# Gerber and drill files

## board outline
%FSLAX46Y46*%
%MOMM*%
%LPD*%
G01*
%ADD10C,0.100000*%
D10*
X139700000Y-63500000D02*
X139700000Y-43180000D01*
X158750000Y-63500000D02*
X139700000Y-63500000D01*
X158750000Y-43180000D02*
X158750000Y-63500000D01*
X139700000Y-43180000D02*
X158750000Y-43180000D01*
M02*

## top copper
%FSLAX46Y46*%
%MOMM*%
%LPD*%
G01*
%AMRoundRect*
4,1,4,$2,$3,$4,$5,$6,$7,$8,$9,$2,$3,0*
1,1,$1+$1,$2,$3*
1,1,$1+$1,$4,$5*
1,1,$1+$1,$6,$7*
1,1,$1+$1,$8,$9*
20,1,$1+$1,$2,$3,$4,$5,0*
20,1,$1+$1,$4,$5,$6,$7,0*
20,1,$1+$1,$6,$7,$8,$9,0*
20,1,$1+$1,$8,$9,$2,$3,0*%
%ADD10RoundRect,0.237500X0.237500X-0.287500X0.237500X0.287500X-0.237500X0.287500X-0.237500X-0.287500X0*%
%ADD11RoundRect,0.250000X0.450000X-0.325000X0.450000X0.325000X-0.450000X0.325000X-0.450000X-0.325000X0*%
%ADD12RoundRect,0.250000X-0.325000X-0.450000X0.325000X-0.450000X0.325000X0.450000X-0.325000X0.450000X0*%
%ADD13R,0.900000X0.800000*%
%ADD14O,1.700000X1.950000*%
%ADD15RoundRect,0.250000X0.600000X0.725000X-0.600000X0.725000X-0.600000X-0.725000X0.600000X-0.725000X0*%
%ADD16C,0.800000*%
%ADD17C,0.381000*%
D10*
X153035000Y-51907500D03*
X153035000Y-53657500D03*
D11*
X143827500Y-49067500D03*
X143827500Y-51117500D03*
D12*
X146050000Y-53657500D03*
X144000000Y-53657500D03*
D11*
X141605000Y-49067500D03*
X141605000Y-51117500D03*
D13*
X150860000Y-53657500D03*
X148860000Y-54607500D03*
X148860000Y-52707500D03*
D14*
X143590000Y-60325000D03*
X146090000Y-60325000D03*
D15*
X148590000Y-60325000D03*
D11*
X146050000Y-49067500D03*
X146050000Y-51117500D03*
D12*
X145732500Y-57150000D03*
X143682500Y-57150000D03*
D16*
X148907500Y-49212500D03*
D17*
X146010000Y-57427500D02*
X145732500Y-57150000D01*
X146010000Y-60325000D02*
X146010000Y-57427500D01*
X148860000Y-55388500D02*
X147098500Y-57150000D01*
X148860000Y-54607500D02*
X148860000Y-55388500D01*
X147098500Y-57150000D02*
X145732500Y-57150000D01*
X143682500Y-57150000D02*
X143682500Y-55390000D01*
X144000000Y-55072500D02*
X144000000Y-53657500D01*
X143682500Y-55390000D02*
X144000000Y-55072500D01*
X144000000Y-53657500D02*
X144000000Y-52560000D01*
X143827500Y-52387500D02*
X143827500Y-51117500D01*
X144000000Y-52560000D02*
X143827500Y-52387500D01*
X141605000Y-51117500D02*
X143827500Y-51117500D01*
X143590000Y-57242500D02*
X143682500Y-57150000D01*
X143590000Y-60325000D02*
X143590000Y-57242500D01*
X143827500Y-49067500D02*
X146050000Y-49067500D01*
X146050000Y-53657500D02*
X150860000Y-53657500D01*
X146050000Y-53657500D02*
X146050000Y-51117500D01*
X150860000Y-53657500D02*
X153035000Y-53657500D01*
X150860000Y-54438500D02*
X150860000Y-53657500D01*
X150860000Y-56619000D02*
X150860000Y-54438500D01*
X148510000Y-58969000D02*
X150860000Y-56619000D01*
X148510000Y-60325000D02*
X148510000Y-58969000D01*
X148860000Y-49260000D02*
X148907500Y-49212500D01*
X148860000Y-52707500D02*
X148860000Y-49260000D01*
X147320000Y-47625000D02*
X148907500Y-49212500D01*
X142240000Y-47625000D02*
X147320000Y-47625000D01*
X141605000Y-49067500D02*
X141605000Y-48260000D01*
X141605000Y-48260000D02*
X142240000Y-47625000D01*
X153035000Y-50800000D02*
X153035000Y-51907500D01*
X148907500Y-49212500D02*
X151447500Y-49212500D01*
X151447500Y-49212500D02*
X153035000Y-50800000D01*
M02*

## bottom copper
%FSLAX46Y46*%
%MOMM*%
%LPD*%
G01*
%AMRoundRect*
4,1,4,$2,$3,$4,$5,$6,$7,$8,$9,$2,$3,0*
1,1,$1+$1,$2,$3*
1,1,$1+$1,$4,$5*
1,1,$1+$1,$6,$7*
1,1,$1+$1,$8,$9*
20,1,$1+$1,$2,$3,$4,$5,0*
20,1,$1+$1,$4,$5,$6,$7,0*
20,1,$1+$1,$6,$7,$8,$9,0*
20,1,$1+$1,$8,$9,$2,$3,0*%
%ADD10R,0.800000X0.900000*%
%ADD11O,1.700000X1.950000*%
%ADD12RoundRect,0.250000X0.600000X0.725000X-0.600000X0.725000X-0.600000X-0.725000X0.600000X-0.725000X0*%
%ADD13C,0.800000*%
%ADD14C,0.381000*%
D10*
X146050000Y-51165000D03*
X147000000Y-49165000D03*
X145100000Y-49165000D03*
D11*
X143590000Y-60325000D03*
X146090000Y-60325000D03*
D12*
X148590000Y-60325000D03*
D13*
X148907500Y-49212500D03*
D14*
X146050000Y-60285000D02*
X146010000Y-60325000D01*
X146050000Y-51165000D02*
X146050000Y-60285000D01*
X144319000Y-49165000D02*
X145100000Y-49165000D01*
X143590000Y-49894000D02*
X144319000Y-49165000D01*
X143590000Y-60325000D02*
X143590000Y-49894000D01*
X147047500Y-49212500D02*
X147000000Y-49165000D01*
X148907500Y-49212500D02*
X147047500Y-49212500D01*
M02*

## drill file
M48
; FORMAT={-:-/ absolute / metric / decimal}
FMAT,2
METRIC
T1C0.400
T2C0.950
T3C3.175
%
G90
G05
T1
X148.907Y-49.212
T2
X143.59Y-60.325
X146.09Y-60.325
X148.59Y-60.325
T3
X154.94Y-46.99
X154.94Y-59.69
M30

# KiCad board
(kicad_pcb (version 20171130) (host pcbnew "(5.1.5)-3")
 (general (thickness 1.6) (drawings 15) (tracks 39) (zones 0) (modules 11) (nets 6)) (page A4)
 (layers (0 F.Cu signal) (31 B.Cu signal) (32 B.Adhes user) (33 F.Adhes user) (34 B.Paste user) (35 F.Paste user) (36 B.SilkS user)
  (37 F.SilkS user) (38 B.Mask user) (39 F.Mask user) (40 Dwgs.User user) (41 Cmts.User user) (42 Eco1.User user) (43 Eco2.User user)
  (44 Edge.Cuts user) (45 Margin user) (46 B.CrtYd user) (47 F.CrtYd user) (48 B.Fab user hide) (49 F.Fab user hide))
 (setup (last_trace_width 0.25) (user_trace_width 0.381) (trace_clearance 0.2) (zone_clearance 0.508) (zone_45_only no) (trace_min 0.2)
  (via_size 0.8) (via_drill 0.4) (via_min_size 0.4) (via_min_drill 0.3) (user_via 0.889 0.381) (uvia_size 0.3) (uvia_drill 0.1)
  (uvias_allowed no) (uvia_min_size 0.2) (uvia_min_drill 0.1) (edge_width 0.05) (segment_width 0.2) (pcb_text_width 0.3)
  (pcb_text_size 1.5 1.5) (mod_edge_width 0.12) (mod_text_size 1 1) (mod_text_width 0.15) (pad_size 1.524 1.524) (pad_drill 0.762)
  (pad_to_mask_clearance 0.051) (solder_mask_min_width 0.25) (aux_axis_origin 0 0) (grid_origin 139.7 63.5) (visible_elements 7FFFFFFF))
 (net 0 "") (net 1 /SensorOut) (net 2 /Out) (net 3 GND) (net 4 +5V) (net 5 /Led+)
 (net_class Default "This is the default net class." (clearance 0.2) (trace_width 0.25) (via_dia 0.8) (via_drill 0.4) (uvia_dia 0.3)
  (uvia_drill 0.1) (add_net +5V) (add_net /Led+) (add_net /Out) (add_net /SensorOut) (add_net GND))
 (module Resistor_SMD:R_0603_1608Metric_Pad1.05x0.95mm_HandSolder (layer F.Cu) (at 153.035 52.7825 90)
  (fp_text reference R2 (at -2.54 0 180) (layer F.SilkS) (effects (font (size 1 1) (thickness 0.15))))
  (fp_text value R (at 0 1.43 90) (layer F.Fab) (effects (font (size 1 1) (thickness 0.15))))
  (pad 2 smd roundrect (at 0.875 0 90) (size 1.05 0.95) (layers F.Cu F.Paste F.Mask) (roundrect_rratio 0.25) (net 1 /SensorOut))
  (pad 1 smd roundrect (at -0.875 0 90) (size 1.05 0.95) (layers F.Cu F.Paste F.Mask) (roundrect_rratio 0.25) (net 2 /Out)))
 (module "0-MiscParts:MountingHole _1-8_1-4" (layer F.Cu) (at 154.94 59.69)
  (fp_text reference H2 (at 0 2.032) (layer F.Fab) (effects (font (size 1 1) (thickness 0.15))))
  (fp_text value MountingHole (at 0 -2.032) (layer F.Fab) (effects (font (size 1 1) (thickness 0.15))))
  (pad "" np_thru_hole circle (at 0 0) (size 3.175 3.175) (drill 3.175) (layers *.Cu *.Mask)))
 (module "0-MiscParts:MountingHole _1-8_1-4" (layer F.Cu) (at 154.94 46.99)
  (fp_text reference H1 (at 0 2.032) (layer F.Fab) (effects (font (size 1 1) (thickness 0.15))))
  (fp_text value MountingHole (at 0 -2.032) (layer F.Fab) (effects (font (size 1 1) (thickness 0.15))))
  (pad "" np_thru_hole circle (at 0 0) (size 3.175 3.175) (drill 3.175) (layers *.Cu *.Mask)))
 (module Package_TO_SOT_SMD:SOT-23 (layer B.Cu) (at 146.05 50.165 270)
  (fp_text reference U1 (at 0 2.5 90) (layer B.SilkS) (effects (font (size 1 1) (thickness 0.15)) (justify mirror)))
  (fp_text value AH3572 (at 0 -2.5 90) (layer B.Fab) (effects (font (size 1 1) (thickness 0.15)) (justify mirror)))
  (pad 3 smd rect (at 1 0 270) (size 0.9 0.8) (layers B.Cu B.Paste B.Mask) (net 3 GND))
  (pad 2 smd rect (at -1 -0.95 270) (size 0.9 0.8) (layers B.Cu B.Paste B.Mask) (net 1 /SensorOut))
  (pad 1 smd rect (at -1 0.95 270) (size 0.9 0.8) (layers B.Cu B.Paste B.Mask) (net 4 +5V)))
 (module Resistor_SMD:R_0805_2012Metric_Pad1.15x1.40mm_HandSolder (layer F.Cu) (at 143.8275 50.0925 90)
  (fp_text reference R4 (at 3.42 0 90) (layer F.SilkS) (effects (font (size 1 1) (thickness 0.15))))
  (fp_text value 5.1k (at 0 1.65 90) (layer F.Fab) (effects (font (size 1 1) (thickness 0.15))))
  (pad 2 smd roundrect (at 1.025 0 90) (size 1.15 1.4) (layers F.Cu F.Paste F.Mask) (roundrect_rratio 0.217391) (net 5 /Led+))
  (pad 1 smd roundrect (at -1.025 0 90) (size 1.15 1.4) (layers F.Cu F.Paste F.Mask) (roundrect_rratio 0.217391) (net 4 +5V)))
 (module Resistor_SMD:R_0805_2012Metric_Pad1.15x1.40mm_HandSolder (layer F.Cu) (at 145.025 53.6575)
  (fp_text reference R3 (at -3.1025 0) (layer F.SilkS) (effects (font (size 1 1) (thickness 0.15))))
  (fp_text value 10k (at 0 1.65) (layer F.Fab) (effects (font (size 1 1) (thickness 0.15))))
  (pad 2 smd roundrect (at 1.025 0) (size 1.15 1.4) (layers F.Cu F.Paste F.Mask) (roundrect_rratio 0.217391) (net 2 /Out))
  (pad 1 smd roundrect (at -1.025 0) (size 1.15 1.4) (layers F.Cu F.Paste F.Mask) (roundrect_rratio 0.217391) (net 4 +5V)))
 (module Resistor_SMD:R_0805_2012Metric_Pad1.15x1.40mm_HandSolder (layer F.Cu) (at 141.605 50.0925 90)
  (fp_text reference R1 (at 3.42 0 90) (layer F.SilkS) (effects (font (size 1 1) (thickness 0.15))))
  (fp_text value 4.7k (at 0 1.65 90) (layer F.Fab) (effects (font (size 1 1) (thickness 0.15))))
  (pad 2 smd roundrect (at 1.025 0 90) (size 1.15 1.4) (layers F.Cu F.Paste F.Mask) (roundrect_rratio 0.217391) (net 1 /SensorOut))
  (pad 1 smd roundrect (at -1.025 0 90) (size 1.15 1.4) (layers F.Cu F.Paste F.Mask) (roundrect_rratio 0.217391) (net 4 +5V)))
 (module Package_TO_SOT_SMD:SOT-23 (layer F.Cu) (at 149.86 53.6575)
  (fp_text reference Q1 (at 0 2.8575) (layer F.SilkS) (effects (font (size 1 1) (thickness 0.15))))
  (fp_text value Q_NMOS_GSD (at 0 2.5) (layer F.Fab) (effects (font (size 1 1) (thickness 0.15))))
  (pad 3 smd rect (at 1 0) (size 0.9 0.8) (layers F.Cu F.Paste F.Mask) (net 2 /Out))
  (pad 2 smd rect (at -1 0.95) (size 0.9 0.8) (layers F.Cu F.Paste F.Mask) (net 3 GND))
  (pad 1 smd rect (at -1 -0.95) (size 0.9 0.8) (layers F.Cu F.Paste F.Mask) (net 1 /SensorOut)))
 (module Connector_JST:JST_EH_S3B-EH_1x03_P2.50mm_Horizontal (layer F.Cu) (at 148.59 60.325 180)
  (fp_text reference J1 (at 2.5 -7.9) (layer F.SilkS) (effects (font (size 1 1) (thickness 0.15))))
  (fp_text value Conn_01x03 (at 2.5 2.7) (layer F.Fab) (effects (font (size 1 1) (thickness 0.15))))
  (pad 3 thru_hole oval (at 5 0 180) (size 1.7 1.95) (drill 0.95) (layers *.Cu *.Mask) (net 4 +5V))
  (pad 2 thru_hole oval (at 2.5 0 180) (size 1.7 1.95) (drill 0.95) (layers *.Cu *.Mask) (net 3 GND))
  (pad 1 thru_hole roundrect (at 0 0 180) (size 1.7 1.95) (drill 0.95) (layers *.Cu *.Mask) (roundrect_rratio 0.147059) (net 2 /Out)))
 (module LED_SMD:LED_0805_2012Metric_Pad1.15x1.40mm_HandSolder (layer F.Cu) (at 146.05 50.0925 90)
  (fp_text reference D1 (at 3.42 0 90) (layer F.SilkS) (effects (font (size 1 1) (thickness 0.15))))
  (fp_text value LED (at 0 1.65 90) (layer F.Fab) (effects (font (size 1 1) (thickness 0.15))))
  (pad 2 smd roundrect (at 1.025 0 90) (size 1.15 1.4) (layers F.Cu F.Paste F.Mask) (roundrect_rratio 0.217391) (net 5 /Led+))
  (pad 1 smd roundrect (at -1.025 0 90) (size 1.15 1.4) (layers F.Cu F.Paste F.Mask) (roundrect_rratio 0.217391) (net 2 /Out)))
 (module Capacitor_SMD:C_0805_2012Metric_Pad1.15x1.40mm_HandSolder (layer F.Cu) (at 144.7075 57.15)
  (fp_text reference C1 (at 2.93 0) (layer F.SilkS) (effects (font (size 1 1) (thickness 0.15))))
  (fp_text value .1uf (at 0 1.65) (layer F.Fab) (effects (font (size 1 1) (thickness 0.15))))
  (pad 2 smd roundrect (at 1.025 0) (size 1.15 1.4) (layers F.Cu F.Paste F.Mask) (roundrect_rratio 0.217391) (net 3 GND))
  (pad 1 smd roundrect (at -1.025 0) (size 1.15 1.4) (layers F.Cu F.Paste F.Mask) (roundrect_rratio 0.217391) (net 4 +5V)))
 (gr_line (start 139.7 63.5) (end 139.7 43.18) (layer Edge.Cuts) (width 0.1))
 (gr_line (start 158.75 63.5) (end 139.7 63.5) (layer Edge.Cuts) (width 0.1))
 (gr_line (start 158.75 43.18) (end 158.75 63.5) (layer Edge.Cuts) (width 0.1))
 (gr_line (start 139.7 43.18) (end 158.75 43.18) (layer Edge.Cuts) (width 0.1))
 (segment (start 146.01 57.4275) (end 145.7325 57.15) (width 0.381) (layer F.Cu) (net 3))
 (segment (start 146.01 60.325) (end 146.01 57.4275) (width 0.381) (layer F.Cu) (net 3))
 (segment (start 148.86 55.3885) (end 147.0985 57.15) (width 0.381) (layer F.Cu) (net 3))
 (segment (start 148.86 54.6075) (end 148.86 55.3885) (width 0.381) (layer F.Cu) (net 3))
 (segment (start 147.0985 57.15) (end 145.7325 57.15) (width 0.381) (layer F.Cu) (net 3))
 (segment (start 146.05 60.285) (end 146.01 60.325) (width 0.381) (layer B.Cu) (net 3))
 (segment (start 146.05 51.165) (end 146.05 60.285) (width 0.381) (layer B.Cu) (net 3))
 (segment (start 143.6825 57.15) (end 143.6825 55.39) (width 0.381) (layer F.Cu) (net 4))
 (segment (start 144 55.0725) (end 144 53.6575) (width 0.381) (layer F.Cu) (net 4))
 (segment (start 143.6825 55.39) (end 144 55.0725) (width 0.381) (layer F.Cu) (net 4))
 (segment (start 144 53.6575) (end 144 52.56) (width 0.381) (layer F.Cu) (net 4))
 (segment (start 143.8275 52.3875) (end 143.8275 51.1175) (width 0.381) (layer F.Cu) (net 4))
 (segment (start 144 52.56) (end 143.8275 52.3875) (width 0.381) (layer F.Cu) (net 4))
 (segment (start 141.605 51.1175) (end 143.8275 51.1175) (width 0.381) (layer F.Cu) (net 4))
 (segment (start 144.319 49.165) (end 145.1 49.165) (width 0.381) (layer B.Cu) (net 4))
 (segment (start 143.59 49.894) (end 144.319 49.165) (width 0.381) (layer B.Cu) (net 4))
 (segment (start 143.59 60.325) (end 143.59 49.894) (width 0.381) (layer B.Cu) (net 4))
 (segment (start 143.59 57.2425) (end 143.6825 57.15) (width 0.381) (layer F.Cu) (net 4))
 (segment (start 143.59 60.325) (end 143.59 57.2425) (width 0.381) (layer F.Cu) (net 4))
 (segment (start 143.8275 49.0675) (end 146.05 49.0675) (width 0.381) (layer F.Cu) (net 5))
 (segment (start 146.05 53.6575) (end 150.86 53.6575) (width 0.381) (layer F.Cu) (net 2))
 (segment (start 146.05 53.6575) (end 146.05 51.1175) (width 0.381) (layer F.Cu) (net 2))
 (segment (start 150.86 53.6575) (end 153.035 53.6575) (width 0.381) (layer F.Cu) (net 2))
 (segment (start 150.86 54.4385) (end 150.86 53.6575) (width 0.381) (layer F.Cu) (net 2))
 (segment (start 150.86 56.619) (end 150.86 54.4385) (width 0.381) (layer F.Cu) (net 2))
 (segment (start 148.51 58.969) (end 150.86 56.619) (width 0.381) (layer F.Cu) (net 2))
 (segment (start 148.51 60.325) (end 148.51 58.969) (width 0.381) (layer F.Cu) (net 2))
 (via (at 148.9075 49.2125) (size 0.8) (drill 0.4) (layers F.Cu B.Cu) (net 1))
 (segment (start 148.86 49.26) (end 148.9075 49.2125) (width 0.381) (layer F.Cu) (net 1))
 (segment (start 148.86 52.7075) (end 148.86 49.26) (width 0.381) (layer F.Cu) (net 1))
 (segment (start 147.0475 49.2125) (end 147 49.165) (width 0.381) (layer B.Cu) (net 1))
 (segment (start 148.9075 49.2125) (end 147.0475 49.2125) (width 0.381) (layer B.Cu) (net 1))
 (segment (start 147.32 47.625) (end 148.9075 49.2125) (width 0.381) (layer F.Cu) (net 1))
 (segment (start 142.24 47.625) (end 147.32 47.625) (width 0.381) (layer F.Cu) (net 1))
 (segment (start 141.605 49.0675) (end 141.605 48.26) (width 0.381) (layer F.Cu) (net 1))
 (segment (start 141.605 48.26) (end 142.24 47.625) (width 0.381) (layer F.Cu) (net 1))
 (segment (start 153.035 50.8) (end 153.035 51.9075) (width 0.381) (layer F.Cu) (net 1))
 (segment (start 148.9075 49.2125) (end 151.4475 49.2125) (width 0.381) (layer F.Cu) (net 1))
 (segment (start 151.4475 49.2125) (end 153.035 50.8) (width 0.381) (layer F.Cu) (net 1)))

